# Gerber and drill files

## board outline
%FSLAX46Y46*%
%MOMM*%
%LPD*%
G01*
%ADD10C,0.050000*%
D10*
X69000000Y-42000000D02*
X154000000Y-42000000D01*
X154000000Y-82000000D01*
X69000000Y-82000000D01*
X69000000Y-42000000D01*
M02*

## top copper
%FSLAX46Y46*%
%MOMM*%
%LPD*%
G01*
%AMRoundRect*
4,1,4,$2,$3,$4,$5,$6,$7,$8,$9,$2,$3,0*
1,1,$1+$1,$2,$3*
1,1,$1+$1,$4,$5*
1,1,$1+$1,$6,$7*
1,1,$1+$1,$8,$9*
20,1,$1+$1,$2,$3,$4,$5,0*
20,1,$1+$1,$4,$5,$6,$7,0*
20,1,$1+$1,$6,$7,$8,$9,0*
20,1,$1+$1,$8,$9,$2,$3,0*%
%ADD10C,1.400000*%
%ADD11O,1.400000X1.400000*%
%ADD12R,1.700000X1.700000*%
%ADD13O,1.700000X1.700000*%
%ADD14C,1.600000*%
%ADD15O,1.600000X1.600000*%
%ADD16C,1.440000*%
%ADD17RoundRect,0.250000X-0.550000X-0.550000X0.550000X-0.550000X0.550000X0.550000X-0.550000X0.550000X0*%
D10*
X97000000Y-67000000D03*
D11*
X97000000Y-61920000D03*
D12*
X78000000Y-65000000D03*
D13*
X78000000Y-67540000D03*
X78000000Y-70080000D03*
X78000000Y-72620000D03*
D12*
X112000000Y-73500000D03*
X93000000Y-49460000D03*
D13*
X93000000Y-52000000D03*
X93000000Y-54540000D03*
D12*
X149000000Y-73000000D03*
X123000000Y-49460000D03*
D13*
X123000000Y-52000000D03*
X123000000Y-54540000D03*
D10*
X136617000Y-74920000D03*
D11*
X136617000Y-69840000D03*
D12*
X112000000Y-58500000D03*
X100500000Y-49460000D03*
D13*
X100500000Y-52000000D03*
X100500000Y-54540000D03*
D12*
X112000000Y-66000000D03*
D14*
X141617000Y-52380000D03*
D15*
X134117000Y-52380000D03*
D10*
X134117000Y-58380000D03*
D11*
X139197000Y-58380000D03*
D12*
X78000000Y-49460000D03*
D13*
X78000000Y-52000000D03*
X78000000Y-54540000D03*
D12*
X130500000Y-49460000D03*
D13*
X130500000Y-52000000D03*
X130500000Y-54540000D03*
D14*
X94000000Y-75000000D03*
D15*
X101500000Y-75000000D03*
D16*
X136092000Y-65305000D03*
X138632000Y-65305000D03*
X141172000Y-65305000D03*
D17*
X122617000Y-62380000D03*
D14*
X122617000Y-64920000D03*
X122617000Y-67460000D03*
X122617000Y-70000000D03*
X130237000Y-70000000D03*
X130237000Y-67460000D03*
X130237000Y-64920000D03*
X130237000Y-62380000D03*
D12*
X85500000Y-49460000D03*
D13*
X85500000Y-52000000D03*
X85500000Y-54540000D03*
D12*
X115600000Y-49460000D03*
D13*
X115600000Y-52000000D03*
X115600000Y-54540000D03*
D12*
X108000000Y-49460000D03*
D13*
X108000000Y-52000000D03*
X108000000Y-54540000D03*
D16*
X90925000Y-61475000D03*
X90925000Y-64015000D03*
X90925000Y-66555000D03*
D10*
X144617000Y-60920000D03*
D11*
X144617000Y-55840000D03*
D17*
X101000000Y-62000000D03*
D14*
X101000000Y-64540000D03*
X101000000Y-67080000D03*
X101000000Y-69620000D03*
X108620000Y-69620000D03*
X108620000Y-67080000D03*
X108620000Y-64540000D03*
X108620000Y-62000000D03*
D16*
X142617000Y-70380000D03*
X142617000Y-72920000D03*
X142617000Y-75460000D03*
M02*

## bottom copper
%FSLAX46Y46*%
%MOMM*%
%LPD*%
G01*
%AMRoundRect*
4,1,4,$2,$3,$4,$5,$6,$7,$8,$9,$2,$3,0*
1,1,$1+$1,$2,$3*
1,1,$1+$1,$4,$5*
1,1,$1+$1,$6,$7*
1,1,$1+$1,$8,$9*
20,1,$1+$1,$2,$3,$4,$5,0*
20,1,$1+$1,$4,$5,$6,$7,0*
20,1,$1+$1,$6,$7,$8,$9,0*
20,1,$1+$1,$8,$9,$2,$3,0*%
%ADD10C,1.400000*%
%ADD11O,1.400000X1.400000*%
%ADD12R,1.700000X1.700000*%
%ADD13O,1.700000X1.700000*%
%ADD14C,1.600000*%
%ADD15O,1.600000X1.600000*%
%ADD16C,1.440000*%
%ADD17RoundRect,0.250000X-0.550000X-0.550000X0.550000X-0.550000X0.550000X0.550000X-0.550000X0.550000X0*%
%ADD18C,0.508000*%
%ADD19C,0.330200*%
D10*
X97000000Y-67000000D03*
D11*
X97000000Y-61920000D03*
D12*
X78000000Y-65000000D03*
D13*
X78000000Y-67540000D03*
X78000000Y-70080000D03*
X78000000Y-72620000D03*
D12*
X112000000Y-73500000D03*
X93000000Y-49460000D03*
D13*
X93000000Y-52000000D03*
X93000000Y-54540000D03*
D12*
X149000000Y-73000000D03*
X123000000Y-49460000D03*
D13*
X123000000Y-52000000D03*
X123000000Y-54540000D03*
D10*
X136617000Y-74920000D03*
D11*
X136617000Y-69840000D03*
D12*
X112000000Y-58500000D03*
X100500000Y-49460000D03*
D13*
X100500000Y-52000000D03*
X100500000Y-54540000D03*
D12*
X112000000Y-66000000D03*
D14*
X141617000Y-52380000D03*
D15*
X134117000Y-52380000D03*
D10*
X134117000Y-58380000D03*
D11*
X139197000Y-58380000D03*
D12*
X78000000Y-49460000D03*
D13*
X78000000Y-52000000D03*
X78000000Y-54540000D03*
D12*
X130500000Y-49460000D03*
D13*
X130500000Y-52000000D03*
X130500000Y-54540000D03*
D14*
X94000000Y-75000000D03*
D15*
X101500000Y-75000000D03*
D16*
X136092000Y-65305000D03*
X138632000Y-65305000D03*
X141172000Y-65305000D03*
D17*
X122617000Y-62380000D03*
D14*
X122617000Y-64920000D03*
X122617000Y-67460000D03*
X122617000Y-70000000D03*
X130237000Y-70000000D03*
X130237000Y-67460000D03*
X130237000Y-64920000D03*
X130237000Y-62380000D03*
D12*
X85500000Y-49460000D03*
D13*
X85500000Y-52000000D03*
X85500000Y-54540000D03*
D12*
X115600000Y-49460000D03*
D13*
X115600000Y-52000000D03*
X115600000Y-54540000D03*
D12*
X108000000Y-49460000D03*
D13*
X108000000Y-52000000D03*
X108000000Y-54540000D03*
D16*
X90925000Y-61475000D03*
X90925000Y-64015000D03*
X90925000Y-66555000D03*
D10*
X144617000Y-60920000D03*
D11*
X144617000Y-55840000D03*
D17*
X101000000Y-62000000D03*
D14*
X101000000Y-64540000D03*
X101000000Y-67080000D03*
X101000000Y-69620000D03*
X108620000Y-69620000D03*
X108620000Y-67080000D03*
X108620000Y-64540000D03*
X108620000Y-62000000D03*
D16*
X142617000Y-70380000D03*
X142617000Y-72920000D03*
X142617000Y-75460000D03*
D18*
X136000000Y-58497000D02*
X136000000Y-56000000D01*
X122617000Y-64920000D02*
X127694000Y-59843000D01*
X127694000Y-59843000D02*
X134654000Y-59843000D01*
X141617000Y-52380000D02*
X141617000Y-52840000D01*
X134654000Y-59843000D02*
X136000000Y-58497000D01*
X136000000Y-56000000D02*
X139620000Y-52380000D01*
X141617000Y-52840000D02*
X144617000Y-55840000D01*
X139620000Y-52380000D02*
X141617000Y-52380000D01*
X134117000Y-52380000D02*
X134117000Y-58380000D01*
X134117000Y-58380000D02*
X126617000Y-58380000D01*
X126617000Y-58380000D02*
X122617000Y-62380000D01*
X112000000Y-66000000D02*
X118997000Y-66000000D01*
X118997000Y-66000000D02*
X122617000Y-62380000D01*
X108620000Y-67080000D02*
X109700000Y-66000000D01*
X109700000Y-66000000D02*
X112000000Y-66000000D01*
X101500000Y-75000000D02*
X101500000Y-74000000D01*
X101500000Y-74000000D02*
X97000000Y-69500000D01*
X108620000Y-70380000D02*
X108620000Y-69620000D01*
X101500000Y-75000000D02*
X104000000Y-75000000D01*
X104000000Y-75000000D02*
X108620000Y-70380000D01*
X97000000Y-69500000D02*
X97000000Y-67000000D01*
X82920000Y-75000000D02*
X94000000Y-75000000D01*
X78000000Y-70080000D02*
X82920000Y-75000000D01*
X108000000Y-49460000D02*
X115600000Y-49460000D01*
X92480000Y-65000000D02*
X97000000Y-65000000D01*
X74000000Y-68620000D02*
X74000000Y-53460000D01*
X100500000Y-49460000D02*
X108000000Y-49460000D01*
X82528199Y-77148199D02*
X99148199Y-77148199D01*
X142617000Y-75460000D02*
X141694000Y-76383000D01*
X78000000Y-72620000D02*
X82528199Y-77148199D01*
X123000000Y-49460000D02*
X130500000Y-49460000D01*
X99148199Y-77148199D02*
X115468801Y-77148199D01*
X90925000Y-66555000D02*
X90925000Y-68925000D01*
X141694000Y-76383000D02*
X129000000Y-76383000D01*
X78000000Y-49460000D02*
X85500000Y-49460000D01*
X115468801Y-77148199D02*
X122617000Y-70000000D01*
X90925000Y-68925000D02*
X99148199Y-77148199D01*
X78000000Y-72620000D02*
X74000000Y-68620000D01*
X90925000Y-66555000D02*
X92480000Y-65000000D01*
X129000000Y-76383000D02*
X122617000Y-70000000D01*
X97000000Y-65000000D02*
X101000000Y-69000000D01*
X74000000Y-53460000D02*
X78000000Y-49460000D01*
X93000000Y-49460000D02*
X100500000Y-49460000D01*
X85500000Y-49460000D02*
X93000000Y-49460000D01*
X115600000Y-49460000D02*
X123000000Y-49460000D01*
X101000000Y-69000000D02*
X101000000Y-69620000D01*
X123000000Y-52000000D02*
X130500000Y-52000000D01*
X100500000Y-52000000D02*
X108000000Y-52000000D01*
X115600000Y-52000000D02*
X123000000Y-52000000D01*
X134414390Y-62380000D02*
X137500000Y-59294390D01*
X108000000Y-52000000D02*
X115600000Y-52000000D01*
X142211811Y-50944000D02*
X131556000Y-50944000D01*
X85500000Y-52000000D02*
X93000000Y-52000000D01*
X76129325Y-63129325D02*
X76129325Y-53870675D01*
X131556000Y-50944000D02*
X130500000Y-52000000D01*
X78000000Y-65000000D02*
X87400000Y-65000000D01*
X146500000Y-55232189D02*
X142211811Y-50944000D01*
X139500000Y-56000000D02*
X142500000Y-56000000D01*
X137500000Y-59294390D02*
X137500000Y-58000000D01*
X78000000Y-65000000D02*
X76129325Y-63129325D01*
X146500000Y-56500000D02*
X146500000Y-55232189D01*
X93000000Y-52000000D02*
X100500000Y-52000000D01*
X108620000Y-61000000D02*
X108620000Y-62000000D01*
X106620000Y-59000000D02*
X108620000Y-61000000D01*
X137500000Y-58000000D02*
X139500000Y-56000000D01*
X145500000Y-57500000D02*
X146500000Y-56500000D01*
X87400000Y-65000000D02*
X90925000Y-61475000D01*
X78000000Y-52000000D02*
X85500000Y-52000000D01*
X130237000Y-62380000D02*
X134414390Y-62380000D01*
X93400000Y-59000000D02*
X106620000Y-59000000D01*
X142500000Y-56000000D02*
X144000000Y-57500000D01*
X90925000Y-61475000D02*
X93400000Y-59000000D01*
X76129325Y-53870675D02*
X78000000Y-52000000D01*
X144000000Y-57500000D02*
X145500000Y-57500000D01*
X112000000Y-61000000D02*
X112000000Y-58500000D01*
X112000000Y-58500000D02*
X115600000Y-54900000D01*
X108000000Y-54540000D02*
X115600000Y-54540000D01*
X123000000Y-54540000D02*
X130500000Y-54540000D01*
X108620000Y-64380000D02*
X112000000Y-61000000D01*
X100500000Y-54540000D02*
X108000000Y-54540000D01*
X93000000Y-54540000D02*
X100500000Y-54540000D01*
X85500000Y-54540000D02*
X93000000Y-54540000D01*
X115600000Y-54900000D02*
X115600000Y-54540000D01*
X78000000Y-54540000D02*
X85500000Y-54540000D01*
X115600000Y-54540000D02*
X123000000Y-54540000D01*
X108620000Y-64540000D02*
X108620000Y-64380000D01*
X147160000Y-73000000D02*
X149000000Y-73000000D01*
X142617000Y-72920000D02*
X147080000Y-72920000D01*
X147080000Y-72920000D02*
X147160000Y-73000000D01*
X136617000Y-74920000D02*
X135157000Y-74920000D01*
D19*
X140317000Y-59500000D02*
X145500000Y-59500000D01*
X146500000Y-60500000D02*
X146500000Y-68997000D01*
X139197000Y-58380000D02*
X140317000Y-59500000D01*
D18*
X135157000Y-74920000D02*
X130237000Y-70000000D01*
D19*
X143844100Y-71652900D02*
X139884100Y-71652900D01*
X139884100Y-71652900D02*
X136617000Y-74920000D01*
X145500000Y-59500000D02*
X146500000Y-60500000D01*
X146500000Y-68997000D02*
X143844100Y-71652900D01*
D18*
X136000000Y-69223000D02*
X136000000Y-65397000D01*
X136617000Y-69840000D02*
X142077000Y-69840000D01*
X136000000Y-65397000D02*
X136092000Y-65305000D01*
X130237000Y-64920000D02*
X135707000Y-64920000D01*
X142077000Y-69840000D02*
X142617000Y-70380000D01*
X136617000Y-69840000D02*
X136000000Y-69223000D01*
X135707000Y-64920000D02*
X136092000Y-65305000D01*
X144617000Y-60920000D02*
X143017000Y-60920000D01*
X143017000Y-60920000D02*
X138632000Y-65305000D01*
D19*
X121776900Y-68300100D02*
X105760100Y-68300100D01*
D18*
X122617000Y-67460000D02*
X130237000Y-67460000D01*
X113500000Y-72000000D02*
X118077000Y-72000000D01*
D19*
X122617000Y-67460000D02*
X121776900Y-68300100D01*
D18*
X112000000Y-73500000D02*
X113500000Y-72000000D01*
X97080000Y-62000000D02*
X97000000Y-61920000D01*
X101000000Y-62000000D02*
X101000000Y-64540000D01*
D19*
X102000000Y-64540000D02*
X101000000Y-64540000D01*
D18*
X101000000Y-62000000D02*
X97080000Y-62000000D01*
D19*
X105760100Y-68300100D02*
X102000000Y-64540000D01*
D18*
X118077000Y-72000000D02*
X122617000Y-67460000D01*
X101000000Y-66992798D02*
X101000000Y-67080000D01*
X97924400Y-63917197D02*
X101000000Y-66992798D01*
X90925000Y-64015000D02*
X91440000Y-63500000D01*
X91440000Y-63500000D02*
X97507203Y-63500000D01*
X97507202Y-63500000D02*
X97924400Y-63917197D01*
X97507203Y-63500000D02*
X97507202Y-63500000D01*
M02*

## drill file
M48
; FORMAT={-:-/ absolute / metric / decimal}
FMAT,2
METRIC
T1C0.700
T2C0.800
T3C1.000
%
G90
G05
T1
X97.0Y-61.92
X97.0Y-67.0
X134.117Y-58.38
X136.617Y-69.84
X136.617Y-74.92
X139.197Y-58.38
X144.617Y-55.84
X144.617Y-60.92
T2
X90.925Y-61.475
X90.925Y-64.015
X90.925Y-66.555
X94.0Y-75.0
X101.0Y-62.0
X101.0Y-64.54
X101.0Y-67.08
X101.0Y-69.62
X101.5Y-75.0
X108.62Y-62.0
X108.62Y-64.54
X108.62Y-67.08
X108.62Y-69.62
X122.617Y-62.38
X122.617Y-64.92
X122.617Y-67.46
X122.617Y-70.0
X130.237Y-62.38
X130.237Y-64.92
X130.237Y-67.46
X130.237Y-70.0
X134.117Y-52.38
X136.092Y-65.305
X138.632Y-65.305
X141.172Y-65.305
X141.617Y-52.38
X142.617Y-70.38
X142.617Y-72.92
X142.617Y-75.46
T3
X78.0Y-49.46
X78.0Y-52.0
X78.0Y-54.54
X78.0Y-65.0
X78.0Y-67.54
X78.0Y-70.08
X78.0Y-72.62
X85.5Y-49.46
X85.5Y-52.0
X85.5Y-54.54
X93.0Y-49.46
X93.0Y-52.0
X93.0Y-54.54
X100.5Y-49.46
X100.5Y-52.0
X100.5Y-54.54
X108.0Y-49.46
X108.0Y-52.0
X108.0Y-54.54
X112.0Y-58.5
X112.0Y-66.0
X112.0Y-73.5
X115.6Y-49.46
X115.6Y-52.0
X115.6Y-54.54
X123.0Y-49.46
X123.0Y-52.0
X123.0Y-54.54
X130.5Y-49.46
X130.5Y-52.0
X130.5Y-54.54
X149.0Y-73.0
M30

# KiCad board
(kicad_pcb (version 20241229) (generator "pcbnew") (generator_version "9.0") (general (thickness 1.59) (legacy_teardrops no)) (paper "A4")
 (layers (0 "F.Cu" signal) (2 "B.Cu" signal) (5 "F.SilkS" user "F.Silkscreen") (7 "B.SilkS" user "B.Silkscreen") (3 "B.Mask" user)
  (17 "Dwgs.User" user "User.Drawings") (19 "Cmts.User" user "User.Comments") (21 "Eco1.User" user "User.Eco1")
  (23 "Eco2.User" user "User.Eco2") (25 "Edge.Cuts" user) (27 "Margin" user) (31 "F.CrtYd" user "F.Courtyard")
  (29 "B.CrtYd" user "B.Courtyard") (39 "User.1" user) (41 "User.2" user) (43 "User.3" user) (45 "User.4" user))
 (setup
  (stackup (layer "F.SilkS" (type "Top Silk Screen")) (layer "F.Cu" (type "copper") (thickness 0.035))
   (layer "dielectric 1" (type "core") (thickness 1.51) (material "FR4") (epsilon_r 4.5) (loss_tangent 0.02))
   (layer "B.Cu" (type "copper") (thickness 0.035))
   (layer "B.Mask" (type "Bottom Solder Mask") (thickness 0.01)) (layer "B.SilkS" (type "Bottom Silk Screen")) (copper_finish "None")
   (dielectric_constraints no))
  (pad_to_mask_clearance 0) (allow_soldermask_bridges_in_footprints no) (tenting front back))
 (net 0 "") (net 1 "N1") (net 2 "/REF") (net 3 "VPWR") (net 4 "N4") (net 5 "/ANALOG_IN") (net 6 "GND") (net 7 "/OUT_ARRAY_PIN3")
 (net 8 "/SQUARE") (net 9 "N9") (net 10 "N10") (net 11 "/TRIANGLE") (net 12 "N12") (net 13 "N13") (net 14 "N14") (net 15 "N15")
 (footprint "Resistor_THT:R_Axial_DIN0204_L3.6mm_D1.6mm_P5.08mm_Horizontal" (layer "F.Cu") (at 97 67 90)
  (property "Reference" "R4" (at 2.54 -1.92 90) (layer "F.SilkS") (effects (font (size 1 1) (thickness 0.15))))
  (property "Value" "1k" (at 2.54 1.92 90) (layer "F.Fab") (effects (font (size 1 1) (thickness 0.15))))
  (pad "1" thru_hole circle (at 0 0 90) (size 1.4 1.4) (drill 0.7) (layers "*.Cu" "*.Mask") (remove_unused_layers no) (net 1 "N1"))
  (pad "2" thru_hole oval (at 5.08 0 90) (size 1.4 1.4) (drill 0.7) (layers "*.Cu" "*.Mask") (remove_unused_layers no) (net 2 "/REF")))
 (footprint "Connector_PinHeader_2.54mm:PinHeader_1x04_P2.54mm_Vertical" (layer "F.Cu") (at 78 65)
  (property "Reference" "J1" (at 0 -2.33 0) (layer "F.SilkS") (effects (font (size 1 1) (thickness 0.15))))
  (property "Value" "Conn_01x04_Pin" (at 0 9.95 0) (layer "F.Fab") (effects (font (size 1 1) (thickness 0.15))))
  (pad "1" thru_hole rect (at 0 0) (size 1.7 1.7) (drill 1) (layers "*.Cu" "*.Mask") (remove_unused_layers no) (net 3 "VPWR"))
  (pad "2" thru_hole oval (at 0 2.54) (size 1.7 1.7) (drill 1) (layers "*.Cu" "*.Mask") (remove_unused_layers no) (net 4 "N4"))
  (pad "3" thru_hole oval (at 0 5.08) (size 1.7 1.7) (drill 1) (layers "*.Cu" "*.Mask") (remove_unused_layers no) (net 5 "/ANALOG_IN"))
  (pad "4" thru_hole oval (at 0 7.62) (size 1.7 1.7) (drill 1) (layers "*.Cu" "*.Mask") (remove_unused_layers no) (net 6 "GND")))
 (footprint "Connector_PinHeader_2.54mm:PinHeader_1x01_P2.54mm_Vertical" (layer "F.Cu") (at 112 73.5)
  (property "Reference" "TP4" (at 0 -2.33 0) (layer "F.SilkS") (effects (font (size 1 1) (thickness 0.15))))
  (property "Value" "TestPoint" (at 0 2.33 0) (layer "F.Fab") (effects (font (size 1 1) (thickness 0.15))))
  (pad "1" thru_hole rect (at 0 0) (size 1.7 1.7) (drill 1) (layers "*.Cu" "*.Mask") (remove_unused_layers no) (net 2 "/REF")))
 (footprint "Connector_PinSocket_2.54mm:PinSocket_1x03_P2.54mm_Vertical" (layer "F.Cu") (at 93 49.46)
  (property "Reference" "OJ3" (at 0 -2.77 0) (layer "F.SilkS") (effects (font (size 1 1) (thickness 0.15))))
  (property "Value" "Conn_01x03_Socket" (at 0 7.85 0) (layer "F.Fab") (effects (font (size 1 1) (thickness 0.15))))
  (pad "1" thru_hole rect (at 0 0) (size 1.7 1.7) (drill 1) (layers "*.Cu" "*.Mask") (remove_unused_layers no) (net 6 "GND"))
  (pad "2" thru_hole oval (at 0 2.54) (size 1.7 1.7) (drill 1) (layers "*.Cu" "*.Mask") (remove_unused_layers no) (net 3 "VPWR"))
  (pad "3" thru_hole oval (at 0 5.08) (size 1.7 1.7) (drill 1) (layers "*.Cu" "*.Mask") (remove_unused_layers no) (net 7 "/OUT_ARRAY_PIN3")))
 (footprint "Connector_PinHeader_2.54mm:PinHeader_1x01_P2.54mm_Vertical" (layer "F.Cu") (at 149 73)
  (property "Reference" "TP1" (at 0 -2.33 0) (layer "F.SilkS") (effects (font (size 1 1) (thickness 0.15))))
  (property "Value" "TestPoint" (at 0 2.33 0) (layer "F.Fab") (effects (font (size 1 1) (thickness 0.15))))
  (pad "1" thru_hole rect (at 0 0) (size 1.7 1.7) (drill 1) (layers "*.Cu" "*.Mask") (remove_unused_layers no) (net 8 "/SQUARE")))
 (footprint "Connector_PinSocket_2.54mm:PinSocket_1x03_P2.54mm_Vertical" (layer "F.Cu") (at 123 49.46)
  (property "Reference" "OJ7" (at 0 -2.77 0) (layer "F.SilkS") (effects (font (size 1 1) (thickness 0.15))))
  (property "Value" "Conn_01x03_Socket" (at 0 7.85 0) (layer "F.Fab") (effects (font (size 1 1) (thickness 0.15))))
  (pad "1" thru_hole rect (at 0 0) (size 1.7 1.7) (drill 1) (layers "*.Cu" "*.Mask") (remove_unused_layers no) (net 6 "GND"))
  (pad "2" thru_hole oval (at 0 2.54) (size 1.7 1.7) (drill 1) (layers "*.Cu" "*.Mask") (remove_unused_layers no) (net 3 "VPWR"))
  (pad "3" thru_hole oval (at 0 5.08) (size 1.7 1.7) (drill 1) (layers "*.Cu" "*.Mask") (remove_unused_layers no) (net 7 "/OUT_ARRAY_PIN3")))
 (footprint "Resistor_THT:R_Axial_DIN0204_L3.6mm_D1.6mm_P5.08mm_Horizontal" (layer "F.Cu") (at 136.617 74.92 90)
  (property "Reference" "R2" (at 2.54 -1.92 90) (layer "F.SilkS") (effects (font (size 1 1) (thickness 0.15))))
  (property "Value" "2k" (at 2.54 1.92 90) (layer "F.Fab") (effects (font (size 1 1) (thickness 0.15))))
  (pad "1" thru_hole circle (at 0 0 90) (size 1.4 1.4) (drill 0.7) (layers "*.Cu" "*.Mask") (remove_unused_layers no) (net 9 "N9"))
  (pad "2" thru_hole oval (at 5.08 0 90) (size 1.4 1.4) (drill 0.7) (layers "*.Cu" "*.Mask") (remove_unused_layers no) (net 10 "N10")))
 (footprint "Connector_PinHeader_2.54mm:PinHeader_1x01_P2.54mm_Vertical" (layer "F.Cu") (at 112 58.5)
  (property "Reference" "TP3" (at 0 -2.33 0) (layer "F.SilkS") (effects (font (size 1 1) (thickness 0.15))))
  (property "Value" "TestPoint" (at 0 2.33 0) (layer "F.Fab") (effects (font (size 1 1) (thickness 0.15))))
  (pad "1" thru_hole rect (at 0 0) (size 1.7 1.7) (drill 1) (layers "*.Cu" "*.Mask") (remove_unused_layers no) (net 7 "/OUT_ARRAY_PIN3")))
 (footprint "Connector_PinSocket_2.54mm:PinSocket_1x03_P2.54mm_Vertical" (layer "F.Cu") (at 100.5 49.46)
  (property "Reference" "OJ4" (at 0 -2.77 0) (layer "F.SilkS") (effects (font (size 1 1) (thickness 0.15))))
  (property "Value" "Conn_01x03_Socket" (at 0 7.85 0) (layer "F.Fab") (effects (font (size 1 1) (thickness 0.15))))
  (pad "1" thru_hole rect (at 0 0) (size 1.7 1.7) (drill 1) (layers "*.Cu" "*.Mask") (remove_unused_layers no) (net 6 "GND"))
  (pad "2" thru_hole oval (at 0 2.54) (size 1.7 1.7) (drill 1) (layers "*.Cu" "*.Mask") (remove_unused_layers no) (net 3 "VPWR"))
  (pad "3" thru_hole oval (at 0 5.08) (size 1.7 1.7) (drill 1) (layers "*.Cu" "*.Mask") (remove_unused_layers no) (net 7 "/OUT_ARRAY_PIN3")))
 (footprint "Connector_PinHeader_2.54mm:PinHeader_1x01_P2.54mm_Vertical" (layer "F.Cu") (at 112 66)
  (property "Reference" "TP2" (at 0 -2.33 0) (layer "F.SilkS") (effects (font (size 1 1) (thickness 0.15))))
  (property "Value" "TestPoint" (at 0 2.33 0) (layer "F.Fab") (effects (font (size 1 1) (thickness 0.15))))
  (pad "1" thru_hole rect (at 0 0) (size 1.7 1.7) (drill 1) (layers "*.Cu" "*.Mask") (remove_unused_layers no) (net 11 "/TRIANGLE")))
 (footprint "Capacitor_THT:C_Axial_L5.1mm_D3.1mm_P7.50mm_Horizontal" (layer "F.Cu") (at 141.617 52.38 180)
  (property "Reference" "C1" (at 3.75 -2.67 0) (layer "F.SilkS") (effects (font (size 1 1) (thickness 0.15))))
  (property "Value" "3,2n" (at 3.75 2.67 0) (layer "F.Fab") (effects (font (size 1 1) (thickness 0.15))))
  (pad "1" thru_hole circle (at 0 0 180) (size 1.6 1.6) (drill 0.8) (layers "*.Cu" "*.Mask") (remove_unused_layers no) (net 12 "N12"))
  (pad "2" thru_hole oval (at 7.5 0 180) (size 1.6 1.6) (drill 0.8) (layers "*.Cu" "*.Mask") (remove_unused_layers no) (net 11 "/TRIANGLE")))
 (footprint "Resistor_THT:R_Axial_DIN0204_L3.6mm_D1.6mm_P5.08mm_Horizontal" (layer "F.Cu") (at 134.117 58.38)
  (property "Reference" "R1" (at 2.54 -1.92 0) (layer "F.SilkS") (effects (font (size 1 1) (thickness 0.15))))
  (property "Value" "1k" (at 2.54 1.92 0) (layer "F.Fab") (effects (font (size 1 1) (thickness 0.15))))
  (pad "1" thru_hole circle (at 0 0) (size 1.4 1.4) (drill 0.7) (layers "*.Cu" "*.Mask") (remove_unused_layers no) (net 11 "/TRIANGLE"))
  (pad "2" thru_hole oval (at 5.08 0) (size 1.4 1.4) (drill 0.7) (layers "*.Cu" "*.Mask") (remove_unused_layers no) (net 9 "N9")))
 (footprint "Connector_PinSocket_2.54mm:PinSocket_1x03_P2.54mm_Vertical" (layer "F.Cu") (at 78 49.46)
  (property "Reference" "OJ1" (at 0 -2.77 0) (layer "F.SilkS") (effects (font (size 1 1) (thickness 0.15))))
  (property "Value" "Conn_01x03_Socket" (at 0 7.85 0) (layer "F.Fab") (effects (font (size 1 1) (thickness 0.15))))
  (pad "1" thru_hole rect (at 0 0) (size 1.7 1.7) (drill 1) (layers "*.Cu" "*.Mask") (remove_unused_layers no) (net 6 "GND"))
  (pad "2" thru_hole oval (at 0 2.54) (size 1.7 1.7) (drill 1) (layers "*.Cu" "*.Mask") (remove_unused_layers no) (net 3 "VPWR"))
  (pad "3" thru_hole oval (at 0 5.08) (size 1.7 1.7) (drill 1) (layers "*.Cu" "*.Mask") (remove_unused_layers no) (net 7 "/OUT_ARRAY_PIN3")))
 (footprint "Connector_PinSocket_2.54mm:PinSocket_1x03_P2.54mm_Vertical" (layer "F.Cu") (at 130.5 49.46)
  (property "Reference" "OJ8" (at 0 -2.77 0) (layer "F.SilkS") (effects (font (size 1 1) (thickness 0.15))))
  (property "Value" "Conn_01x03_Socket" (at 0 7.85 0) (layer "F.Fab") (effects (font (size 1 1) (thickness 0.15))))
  (pad "1" thru_hole rect (at 0 0) (size 1.7 1.7) (drill 1) (layers "*.Cu" "*.Mask") (remove_unused_layers no) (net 6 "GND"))
  (pad "2" thru_hole oval (at 0 2.54) (size 1.7 1.7) (drill 1) (layers "*.Cu" "*.Mask") (remove_unused_layers no) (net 3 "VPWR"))
  (pad "3" thru_hole oval (at 0 5.08) (size 1.7 1.7) (drill 1) (layers "*.Cu" "*.Mask") (remove_unused_layers no) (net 7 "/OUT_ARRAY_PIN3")))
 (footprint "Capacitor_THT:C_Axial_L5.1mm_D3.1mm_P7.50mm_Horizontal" (layer "F.Cu") (at 94 75)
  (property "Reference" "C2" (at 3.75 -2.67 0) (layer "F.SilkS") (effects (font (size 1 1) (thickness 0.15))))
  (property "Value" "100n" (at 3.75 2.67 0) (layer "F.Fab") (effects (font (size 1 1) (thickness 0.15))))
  (pad "1" thru_hole circle (at 0 0) (size 1.6 1.6) (drill 0.8) (layers "*.Cu" "*.Mask") (remove_unused_layers no) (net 5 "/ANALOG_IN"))
  (pad "2" thru_hole oval (at 7.5 0) (size 1.6 1.6) (drill 0.8) (layers "*.Cu" "*.Mask") (remove_unused_layers no) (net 1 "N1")))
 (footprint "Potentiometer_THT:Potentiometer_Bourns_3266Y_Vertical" (layer "F.Cu") (at 136.092 65.305 180)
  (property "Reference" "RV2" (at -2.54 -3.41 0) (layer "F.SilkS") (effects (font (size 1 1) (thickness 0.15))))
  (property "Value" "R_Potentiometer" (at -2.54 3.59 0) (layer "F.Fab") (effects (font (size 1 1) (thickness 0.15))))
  (pad "1" thru_hole circle (at 0 0 180) (size 1.44 1.44) (drill 0.8) (layers "*.Cu" "*.Mask") (remove_unused_layers no) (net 10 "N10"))
  (pad "2" thru_hole circle (at -2.54 0 180) (size 1.44 1.44) (drill 0.8) (layers "*.Cu" "*.Mask") (remove_unused_layers no) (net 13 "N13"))
  (pad "3" thru_hole circle (at -5.08 0 180) (size 1.44 1.44) (drill 0.8) (layers "*.Cu" "*.Mask") (remove_unused_layers no) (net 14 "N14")))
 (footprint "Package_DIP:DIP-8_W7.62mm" (layer "F.Cu") (at 122.617 62.38)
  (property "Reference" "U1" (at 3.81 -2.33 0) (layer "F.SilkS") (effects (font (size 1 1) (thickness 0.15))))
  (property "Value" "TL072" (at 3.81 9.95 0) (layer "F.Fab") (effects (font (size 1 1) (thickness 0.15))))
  (pad "1" thru_hole roundrect (at 0 0) (size 1.6 1.6) (drill 0.8) (layers "*.Cu" "*.Mask") (remove_unused_layers no)
   (roundrect_rratio 0.15625) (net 11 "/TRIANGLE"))
  (pad "2" thru_hole circle (at 0 2.54) (size 1.6 1.6) (drill 0.8) (layers "*.Cu" "*.Mask") (remove_unused_layers no) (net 12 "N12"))
  (pad "3" thru_hole circle (at 0 5.08) (size 1.6 1.6) (drill 0.8) (layers "*.Cu" "*.Mask") (remove_unused_layers no) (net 2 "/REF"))
  (pad "4" thru_hole circle (at 0 7.62) (size 1.6 1.6) (drill 0.8) (layers "*.Cu" "*.Mask") (remove_unused_layers no) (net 6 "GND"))
  (pad "5" thru_hole circle (at 7.62 7.62) (size 1.6 1.6) (drill 0.8) (layers "*.Cu" "*.Mask") (remove_unused_layers no) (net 9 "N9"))
  (pad "6" thru_hole circle (at 7.62 5.08) (size 1.6 1.6) (drill 0.8) (layers "*.Cu" "*.Mask") (remove_unused_layers no) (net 2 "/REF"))
  (pad "7" thru_hole circle (at 7.62 2.54) (size 1.6 1.6) (drill 0.8) (layers "*.Cu" "*.Mask") (remove_unused_layers no) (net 10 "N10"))
  (pad "8" thru_hole circle (at 7.62 0) (size 1.6 1.6) (drill 0.8) (layers "*.Cu" "*.Mask") (remove_unused_layers no) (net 3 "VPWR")))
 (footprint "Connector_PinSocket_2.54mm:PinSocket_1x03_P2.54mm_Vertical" (layer "F.Cu") (at 85.5 49.46)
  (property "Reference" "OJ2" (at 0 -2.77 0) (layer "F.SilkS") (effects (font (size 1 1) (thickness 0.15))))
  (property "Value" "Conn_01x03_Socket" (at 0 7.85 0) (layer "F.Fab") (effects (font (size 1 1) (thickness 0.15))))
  (pad "1" thru_hole rect (at 0 0) (size 1.7 1.7) (drill 1) (layers "*.Cu" "*.Mask") (remove_unused_layers no) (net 6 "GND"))
  (pad "2" thru_hole oval (at 0 2.54) (size 1.7 1.7) (drill 1) (layers "*.Cu" "*.Mask") (remove_unused_layers no) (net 3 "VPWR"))
  (pad "3" thru_hole oval (at 0 5.08) (size 1.7 1.7) (drill 1) (layers "*.Cu" "*.Mask") (remove_unused_layers no) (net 7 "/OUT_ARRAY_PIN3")))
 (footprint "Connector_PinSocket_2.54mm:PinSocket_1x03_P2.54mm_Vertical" (layer "F.Cu") (at 115.6 49.46)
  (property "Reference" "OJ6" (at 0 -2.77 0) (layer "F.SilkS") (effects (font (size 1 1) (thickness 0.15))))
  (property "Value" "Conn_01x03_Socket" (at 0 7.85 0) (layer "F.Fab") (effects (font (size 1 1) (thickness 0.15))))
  (pad "1" thru_hole rect (at 0 0) (size 1.7 1.7) (drill 1) (layers "*.Cu" "*.Mask") (remove_unused_layers no) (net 6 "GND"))
  (pad "2" thru_hole oval (at 0 2.54) (size 1.7 1.7) (drill 1) (layers "*.Cu" "*.Mask") (remove_unused_layers no) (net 3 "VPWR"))
  (pad "3" thru_hole oval (at 0 5.08) (size 1.7 1.7) (drill 1) (layers "*.Cu" "*.Mask") (remove_unused_layers no) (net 7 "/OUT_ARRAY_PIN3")))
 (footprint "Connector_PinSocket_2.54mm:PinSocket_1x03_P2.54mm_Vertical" (layer "F.Cu") (at 108 49.46)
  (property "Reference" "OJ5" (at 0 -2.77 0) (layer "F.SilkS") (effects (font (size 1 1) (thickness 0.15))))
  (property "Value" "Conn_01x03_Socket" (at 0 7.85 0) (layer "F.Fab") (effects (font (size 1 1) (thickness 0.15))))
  (pad "1" thru_hole rect (at 0 0) (size 1.7 1.7) (drill 1) (layers "*.Cu" "*.Mask") (remove_unused_layers no) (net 6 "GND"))
  (pad "2" thru_hole oval (at 0 2.54) (size 1.7 1.7) (drill 1) (layers "*.Cu" "*.Mask") (remove_unused_layers no) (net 3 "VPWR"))
  (pad "3" thru_hole oval (at 0 5.08) (size 1.7 1.7) (drill 1) (layers "*.Cu" "*.Mask") (remove_unused_layers no) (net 7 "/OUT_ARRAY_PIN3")))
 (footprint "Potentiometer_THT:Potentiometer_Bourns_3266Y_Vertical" (layer "F.Cu") (at 90.925 61.475 90)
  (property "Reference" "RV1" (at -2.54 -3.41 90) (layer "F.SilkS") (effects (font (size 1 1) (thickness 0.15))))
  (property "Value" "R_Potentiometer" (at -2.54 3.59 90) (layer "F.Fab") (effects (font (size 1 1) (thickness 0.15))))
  (pad "1" thru_hole circle (at 0 0 90) (size 1.44 1.44) (drill 0.8) (layers "*.Cu" "*.Mask") (remove_unused_layers no) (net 3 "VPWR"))
  (pad "2" thru_hole circle (at -2.54 0 90) (size 1.44 1.44) (drill 0.8) (layers "*.Cu" "*.Mask") (remove_unused_layers no) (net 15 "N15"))
  (pad "3" thru_hole circle (at -5.08 0 90) (size 1.44 1.44) (drill 0.8) (layers "*.Cu" "*.Mask") (remove_unused_layers no) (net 6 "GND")))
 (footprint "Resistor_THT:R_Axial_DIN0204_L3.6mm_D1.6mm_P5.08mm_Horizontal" (layer "F.Cu") (at 144.617 60.92 90)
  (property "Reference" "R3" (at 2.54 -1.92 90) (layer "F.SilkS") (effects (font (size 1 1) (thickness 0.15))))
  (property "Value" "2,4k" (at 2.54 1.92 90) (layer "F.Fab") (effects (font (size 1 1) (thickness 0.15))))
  (pad "1" thru_hole circle (at 0 0 90) (size 1.4 1.4) (drill 0.7) (layers "*.Cu" "*.Mask") (remove_unused_layers no) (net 13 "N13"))
  (pad "2" thru_hole oval (at 5.08 0 90) (size 1.4 1.4) (drill 0.7) (layers "*.Cu" "*.Mask") (remove_unused_layers no) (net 12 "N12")))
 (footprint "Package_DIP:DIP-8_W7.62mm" (layer "F.Cu") (at 101 62)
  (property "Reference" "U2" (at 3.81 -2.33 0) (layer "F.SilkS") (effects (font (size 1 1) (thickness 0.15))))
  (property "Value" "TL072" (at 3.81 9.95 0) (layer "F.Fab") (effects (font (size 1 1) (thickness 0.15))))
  (pad "1" thru_hole roundrect (at 0 0) (size 1.6 1.6) (drill 0.8) (layers "*.Cu" "*.Mask") (remove_unused_layers no)
   (roundrect_rratio 0.15625) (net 2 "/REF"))
  (pad "2" thru_hole circle (at 0 2.54) (size 1.6 1.6) (drill 0.8) (layers "*.Cu" "*.Mask") (remove_unused_layers no) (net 2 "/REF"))
  (pad "3" thru_hole circle (at 0 5.08) (size 1.6 1.6) (drill 0.8) (layers "*.Cu" "*.Mask") (remove_unused_layers no) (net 15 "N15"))
  (pad "4" thru_hole circle (at 0 7.62) (size 1.6 1.6) (drill 0.8) (layers "*.Cu" "*.Mask") (remove_unused_layers no) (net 6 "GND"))
  (pad "5" thru_hole circle (at 7.62 7.62) (size 1.6 1.6) (drill 0.8) (layers "*.Cu" "*.Mask") (remove_unused_layers no) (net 1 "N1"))
  (pad "6" thru_hole circle (at 7.62 5.08) (size 1.6 1.6) (drill 0.8) (layers "*.Cu" "*.Mask") (remove_unused_layers no)
   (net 11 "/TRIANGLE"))
  (pad "7" thru_hole circle (at 7.62 2.54) (size 1.6 1.6) (drill 0.8) (layers "*.Cu" "*.Mask") (remove_unused_layers no)
   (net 7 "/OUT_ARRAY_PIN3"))
  (pad "8" thru_hole circle (at 7.62 0) (size 1.6 1.6) (drill 0.8) (layers "*.Cu" "*.Mask") (remove_unused_layers no) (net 3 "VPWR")))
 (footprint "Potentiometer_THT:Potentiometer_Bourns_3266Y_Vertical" (layer "F.Cu") (at 142.617 70.38 90)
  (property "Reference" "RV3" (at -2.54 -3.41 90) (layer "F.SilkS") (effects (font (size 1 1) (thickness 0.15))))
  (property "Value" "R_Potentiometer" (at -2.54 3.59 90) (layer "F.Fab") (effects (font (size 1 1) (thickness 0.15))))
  (pad "1" thru_hole circle (at 0 0 90) (size 1.44 1.44) (drill 0.8) (layers "*.Cu" "*.Mask") (remove_unused_layers no) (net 10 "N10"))
  (pad "2" thru_hole circle (at -2.54 0 90) (size 1.44 1.44) (drill 0.8) (layers "*.Cu" "*.Mask") (remove_unused_layers no)
   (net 8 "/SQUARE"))
  (pad "3" thru_hole circle (at -5.08 0 90) (size 1.44 1.44) (drill 0.8) (layers "*.Cu" "*.Mask") (remove_unused_layers no) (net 6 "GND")))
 (gr_rect (start 69 42) (end 154 82) (stroke (width 0.05) (type default)) (fill no) (layer "Edge.Cuts"))
 (segment (start 136 58.497) (end 136 56) (width 0.508) (layer "B.Cu") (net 12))
 (segment (start 122.617 64.92) (end 127.694 59.843) (width 0.508) (layer "B.Cu") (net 12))
 (segment (start 127.694 59.843) (end 134.654 59.843) (width 0.508) (layer "B.Cu") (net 12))
 (segment (start 141.617 52.38) (end 141.617 52.84) (width 0.508) (layer "B.Cu") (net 12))
 (segment (start 134.654 59.843) (end 136 58.497) (width 0.508) (layer "B.Cu") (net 12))
 (segment (start 136 56) (end 139.62 52.38) (width 0.508) (layer "B.Cu") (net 12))
 (segment (start 141.617 52.84) (end 144.617 55.84) (width 0.508) (layer "B.Cu") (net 12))
 (segment (start 139.62 52.38) (end 141.617 52.38) (width 0.508) (layer "B.Cu") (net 12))
 (segment (start 134.117 52.38) (end 134.117 58.38) (width 0.508) (layer "B.Cu") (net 11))
 (segment (start 134.117 58.38) (end 126.617 58.38) (width 0.508) (layer "B.Cu") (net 11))
 (segment (start 126.617 58.38) (end 122.617 62.38) (width 0.508) (layer "B.Cu") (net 11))
 (segment (start 112 66) (end 118.997 66) (width 0.508) (layer "B.Cu") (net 11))
 (segment (start 118.997 66) (end 122.617 62.38) (width 0.508) (layer "B.Cu") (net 11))
 (segment (start 108.62 67.08) (end 109.7 66) (width 0.508) (layer "B.Cu") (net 11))
 (segment (start 109.7 66) (end 112 66) (width 0.508) (layer "B.Cu") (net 11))
 (segment (start 101.5 75) (end 101.5 74) (width 0.508) (layer "B.Cu") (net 1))
 (segment (start 101.5 74) (end 97 69.5) (width 0.508) (layer "B.Cu") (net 1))
 (segment (start 108.62 70.38) (end 108.62 69.62) (width 0.508) (layer "B.Cu") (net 1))
 (segment (start 101.5 75) (end 104 75) (width 0.508) (layer "B.Cu") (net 1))
 (segment (start 104 75) (end 108.62 70.38) (width 0.508) (layer "B.Cu") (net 1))
 (segment (start 97 69.5) (end 97 67) (width 0.508) (layer "B.Cu") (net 1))
 (segment (start 82.92 75) (end 94 75) (width 0.508) (layer "B.Cu") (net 5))
 (segment (start 78 70.08) (end 82.92 75) (width 0.508) (layer "B.Cu") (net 5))
 (segment (start 108 49.46) (end 115.6 49.46) (width 0.508) (layer "B.Cu") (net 6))
 (segment (start 92.48 65) (end 97 65) (width 0.508) (layer "B.Cu") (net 6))
 (segment (start 74 68.62) (end 74 53.46) (width 0.508) (layer "B.Cu") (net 6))
 (segment (start 100.5 49.46) (end 108 49.46) (width 0.508) (layer "B.Cu") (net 6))
 (segment (start 82.528199 77.148199) (end 99.148199 77.148199) (width 0.508) (layer "B.Cu") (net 6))
 (segment (start 142.617 75.46) (end 141.694 76.383) (width 0.508) (layer "B.Cu") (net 6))
 (segment (start 78 72.62) (end 82.528199 77.148199) (width 0.508) (layer "B.Cu") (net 6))
 (segment (start 123 49.46) (end 130.5 49.46) (width 0.508) (layer "B.Cu") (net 6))
 (segment (start 99.148199 77.148199) (end 115.468801 77.148199) (width 0.508) (layer "B.Cu") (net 6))
 (segment (start 90.925 66.555) (end 90.925 68.925) (width 0.508) (layer "B.Cu") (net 6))
 (segment (start 141.694 76.383) (end 129 76.383) (width 0.508) (layer "B.Cu") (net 6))
 (segment (start 78 49.46) (end 85.5 49.46) (width 0.508) (layer "B.Cu") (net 6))
 (segment (start 115.468801 77.148199) (end 122.617 70) (width 0.508) (layer "B.Cu") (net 6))
 (segment (start 90.925 68.925) (end 99.148199 77.148199) (width 0.508) (layer "B.Cu") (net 6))
 (segment (start 78 72.62) (end 74 68.62) (width 0.508) (layer "B.Cu") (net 6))
 (segment (start 90.925 66.555) (end 92.48 65) (width 0.508) (layer "B.Cu") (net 6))
 (segment (start 129 76.383) (end 122.617 70) (width 0.508) (layer "B.Cu") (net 6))
 (segment (start 97 65) (end 101 69) (width 0.508) (layer "B.Cu") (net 6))
 (segment (start 74 53.46) (end 78 49.46) (width 0.508) (layer "B.Cu") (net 6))
 (segment (start 93 49.46) (end 100.5 49.46) (width 0.508) (layer "B.Cu") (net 6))
 (segment (start 85.5 49.46) (end 93 49.46) (width 0.508) (layer "B.Cu") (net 6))
 (segment (start 115.6 49.46) (end 123 49.46) (width 0.508) (layer "B.Cu") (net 6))
 (segment (start 101 69) (end 101 69.62) (width 0.508) (layer "B.Cu") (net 6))
 (segment (start 123 52) (end 130.5 52) (width 0.508) (layer "B.Cu") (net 3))
 (segment (start 100.5 52) (end 108 52) (width 0.508) (layer "B.Cu") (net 3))
 (segment (start 115.6 52) (end 123 52) (width 0.508) (layer "B.Cu") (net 3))
 (segment (start 134.41439 62.38) (end 137.5 59.29439) (width 0.508) (layer "B.Cu") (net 3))
 (segment (start 108 52) (end 115.6 52) (width 0.508) (layer "B.Cu") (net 3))
 (segment (start 142.211811 50.944) (end 131.556 50.944) (width 0.508) (layer "B.Cu") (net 3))
 (segment (start 85.5 52) (end 93 52) (width 0.508) (layer "B.Cu") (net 3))
 (segment (start 76.129325 63.129325) (end 76.129325 53.870675) (width 0.508) (layer "B.Cu") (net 3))
 (segment (start 131.556 50.944) (end 130.5 52) (width 0.508) (layer "B.Cu") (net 3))
 (segment (start 78 65) (end 87.4 65) (width 0.508) (layer "B.Cu") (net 3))
 (segment (start 146.5 55.232189) (end 142.211811 50.944) (width 0.508) (layer "B.Cu") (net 3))
 (segment (start 139.5 56) (end 142.5 56) (width 0.508) (layer "B.Cu") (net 3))
 (segment (start 137.5 59.29439) (end 137.5 58) (width 0.508) (layer "B.Cu") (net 3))
 (segment (start 78 65) (end 76.129325 63.129325) (width 0.508) (layer "B.Cu") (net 3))
 (segment (start 146.5 56.5) (end 146.5 55.232189) (width 0.508) (layer "B.Cu") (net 3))
 (segment (start 93 52) (end 100.5 52) (width 0.508) (layer "B.Cu") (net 3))
 (segment (start 108.62 61) (end 108.62 62) (width 0.508) (layer "B.Cu") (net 3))
 (segment (start 106.62 59) (end 108.62 61) (width 0.508) (layer "B.Cu") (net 3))
 (segment (start 137.5 58) (end 139.5 56) (width 0.508) (layer "B.Cu") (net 3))
 (segment (start 145.5 57.5) (end 146.5 56.5) (width 0.508) (layer "B.Cu") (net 3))
 (segment (start 87.4 65) (end 90.925 61.475) (width 0.508) (layer "B.Cu") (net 3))
 (segment (start 78 52) (end 85.5 52) (width 0.508) (layer "B.Cu") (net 3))
 (segment (start 130.237 62.38) (end 134.41439 62.38) (width 0.508) (layer "B.Cu") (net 3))
 (segment (start 93.4 59) (end 106.62 59) (width 0.508) (layer "B.Cu") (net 3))
 (segment (start 142.5 56) (end 144 57.5) (width 0.508) (layer "B.Cu") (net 3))
 (segment (start 90.925 61.475) (end 93.4 59) (width 0.508) (layer "B.Cu") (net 3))
 (segment (start 76.129325 53.870675) (end 78 52) (width 0.508) (layer "B.Cu") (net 3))
 (segment (start 144 57.5) (end 145.5 57.5) (width 0.508) (layer "B.Cu") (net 3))
 (segment (start 112 61) (end 112 58.5) (width 0.508) (layer "B.Cu") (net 7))
 (segment (start 112 58.5) (end 115.6 54.9) (width 0.508) (layer "B.Cu") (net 7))
 (segment (start 108 54.54) (end 115.6 54.54) (width 0.508) (layer "B.Cu") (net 7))
 (segment (start 123 54.54) (end 130.5 54.54) (width 0.508) (layer "B.Cu") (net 7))
 (segment (start 108.62 64.38) (end 112 61) (width 0.508) (layer "B.Cu") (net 7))
 (segment (start 100.5 54.54) (end 108 54.54) (width 0.508) (layer "B.Cu") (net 7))
 (segment (start 93 54.54) (end 100.5 54.54) (width 0.508) (layer "B.Cu") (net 7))
 (segment (start 85.5 54.54) (end 93 54.54) (width 0.508) (layer "B.Cu") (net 7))
 (segment (start 115.6 54.9) (end 115.6 54.54) (width 0.508) (layer "B.Cu") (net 7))
 (segment (start 78 54.54) (end 85.5 54.54) (width 0.508) (layer "B.Cu") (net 7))
 (segment (start 115.6 54.54) (end 123 54.54) (width 0.508) (layer "B.Cu") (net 7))
 (segment (start 108.62 64.54) (end 108.62 64.38) (width 0.508) (layer "B.Cu") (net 7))
 (segment (start 147.16 73) (end 149 73) (width 0.508) (layer "B.Cu") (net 8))
 (segment (start 142.617 72.92) (end 147.08 72.92) (width 0.508) (layer "B.Cu") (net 8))
 (segment (start 147.08 72.92) (end 147.16 73) (width 0.508) (layer "B.Cu") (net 8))
 (segment (start 136.617 74.92) (end 135.157 74.92) (width 0.508) (layer "B.Cu") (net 9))
 (segment (start 140.317 59.5) (end 145.5 59.5) (width 0.3302) (layer "B.Cu") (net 9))
 (segment (start 146.5 60.5) (end 146.5 68.997) (width 0.3302) (layer "B.Cu") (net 9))
 (segment (start 139.197 58.38) (end 140.317 59.5) (width 0.3302) (layer "B.Cu") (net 9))
 (segment (start 135.157 74.92) (end 130.237 70) (width 0.508) (layer "B.Cu") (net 9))
 (segment (start 143.8441 71.6529) (end 139.8841 71.6529) (width 0.3302) (layer "B.Cu") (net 9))
 (segment (start 139.8841 71.6529) (end 136.617 74.92) (width 0.3302) (layer "B.Cu") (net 9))
 (segment (start 145.5 59.5) (end 146.5 60.5) (width 0.3302) (layer "B.Cu") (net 9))
 (segment (start 146.5 68.997) (end 143.8441 71.6529) (width 0.3302) (layer "B.Cu") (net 9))
 (segment (start 136 69.223) (end 136 65.397) (width 0.508) (layer "B.Cu") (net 10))
 (segment (start 136.617 69.84) (end 142.077 69.84) (width 0.508) (layer "B.Cu") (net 10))
 (segment (start 136 65.397) (end 136.092 65.305) (width 0.508) (layer "B.Cu") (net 10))
 (segment (start 130.237 64.92) (end 135.707 64.92) (width 0.508) (layer "B.Cu") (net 10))
 (segment (start 142.077 69.84) (end 142.617 70.38) (width 0.508) (layer "B.Cu") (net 10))
 (segment (start 136.617 69.84) (end 136 69.223) (width 0.508) (layer "B.Cu") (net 10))
 (segment (start 135.707 64.92) (end 136.092 65.305) (width 0.508) (layer "B.Cu") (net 10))
 (segment (start 144.617 60.92) (end 143.017 60.92) (width 0.508) (layer "B.Cu") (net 13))
 (segment (start 143.017 60.92) (end 138.632 65.305) (width 0.508) (layer "B.Cu") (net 13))
 (segment (start 121.7769 68.3001) (end 105.7601 68.3001) (width 0.3302) (layer "B.Cu") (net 2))
 (segment (start 122.617 67.46) (end 130.237 67.46) (width 0.508) (layer "B.Cu") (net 2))
 (segment (start 113.5 72) (end 118.077 72) (width 0.508) (layer "B.Cu") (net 2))
 (segment (start 122.617 67.46) (end 121.7769 68.3001) (width 0.3302) (layer "B.Cu") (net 2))
 (segment (start 112 73.5) (end 113.5 72) (width 0.508) (layer "B.Cu") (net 2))
 (segment (start 97.08 62) (end 97 61.92) (width 0.508) (layer "B.Cu") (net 2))
 (segment (start 101 62) (end 101 64.54) (width 0.508) (layer "B.Cu") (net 2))
 (segment (start 102 64.54) (end 101 64.54) (width 0.3302) (layer "B.Cu") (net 2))
 (segment (start 101 62) (end 97.08 62) (width 0.508) (layer "B.Cu") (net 2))
 (segment (start 105.7601 68.3001) (end 102 64.54) (width 0.3302) (layer "B.Cu") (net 2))
 (segment (start 118.077 72) (end 122.617 67.46) (width 0.508) (layer "B.Cu") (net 2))
 (segment (start 101 66.992798) (end 101 67.08) (width 0.508) (layer "B.Cu") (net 15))
 (segment (start 97.9244 63.917197) (end 101 66.992798) (width 0.508) (layer "B.Cu") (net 15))
 (segment (start 90.925 64.015) (end 91.44 63.5) (width 0.508) (layer "B.Cu") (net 15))
 (segment (start 91.44 63.5) (end 97.507203 63.5) (width 0.508) (layer "B.Cu") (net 15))
 (segment (start 97.507202 63.5) (end 97.9244 63.917197) (width 0.508) (layer "B.Cu") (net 15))
 (segment (start 97.507203 63.5) (end 97.507202 63.5) (width 0.508) (layer "B.Cu") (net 15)))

